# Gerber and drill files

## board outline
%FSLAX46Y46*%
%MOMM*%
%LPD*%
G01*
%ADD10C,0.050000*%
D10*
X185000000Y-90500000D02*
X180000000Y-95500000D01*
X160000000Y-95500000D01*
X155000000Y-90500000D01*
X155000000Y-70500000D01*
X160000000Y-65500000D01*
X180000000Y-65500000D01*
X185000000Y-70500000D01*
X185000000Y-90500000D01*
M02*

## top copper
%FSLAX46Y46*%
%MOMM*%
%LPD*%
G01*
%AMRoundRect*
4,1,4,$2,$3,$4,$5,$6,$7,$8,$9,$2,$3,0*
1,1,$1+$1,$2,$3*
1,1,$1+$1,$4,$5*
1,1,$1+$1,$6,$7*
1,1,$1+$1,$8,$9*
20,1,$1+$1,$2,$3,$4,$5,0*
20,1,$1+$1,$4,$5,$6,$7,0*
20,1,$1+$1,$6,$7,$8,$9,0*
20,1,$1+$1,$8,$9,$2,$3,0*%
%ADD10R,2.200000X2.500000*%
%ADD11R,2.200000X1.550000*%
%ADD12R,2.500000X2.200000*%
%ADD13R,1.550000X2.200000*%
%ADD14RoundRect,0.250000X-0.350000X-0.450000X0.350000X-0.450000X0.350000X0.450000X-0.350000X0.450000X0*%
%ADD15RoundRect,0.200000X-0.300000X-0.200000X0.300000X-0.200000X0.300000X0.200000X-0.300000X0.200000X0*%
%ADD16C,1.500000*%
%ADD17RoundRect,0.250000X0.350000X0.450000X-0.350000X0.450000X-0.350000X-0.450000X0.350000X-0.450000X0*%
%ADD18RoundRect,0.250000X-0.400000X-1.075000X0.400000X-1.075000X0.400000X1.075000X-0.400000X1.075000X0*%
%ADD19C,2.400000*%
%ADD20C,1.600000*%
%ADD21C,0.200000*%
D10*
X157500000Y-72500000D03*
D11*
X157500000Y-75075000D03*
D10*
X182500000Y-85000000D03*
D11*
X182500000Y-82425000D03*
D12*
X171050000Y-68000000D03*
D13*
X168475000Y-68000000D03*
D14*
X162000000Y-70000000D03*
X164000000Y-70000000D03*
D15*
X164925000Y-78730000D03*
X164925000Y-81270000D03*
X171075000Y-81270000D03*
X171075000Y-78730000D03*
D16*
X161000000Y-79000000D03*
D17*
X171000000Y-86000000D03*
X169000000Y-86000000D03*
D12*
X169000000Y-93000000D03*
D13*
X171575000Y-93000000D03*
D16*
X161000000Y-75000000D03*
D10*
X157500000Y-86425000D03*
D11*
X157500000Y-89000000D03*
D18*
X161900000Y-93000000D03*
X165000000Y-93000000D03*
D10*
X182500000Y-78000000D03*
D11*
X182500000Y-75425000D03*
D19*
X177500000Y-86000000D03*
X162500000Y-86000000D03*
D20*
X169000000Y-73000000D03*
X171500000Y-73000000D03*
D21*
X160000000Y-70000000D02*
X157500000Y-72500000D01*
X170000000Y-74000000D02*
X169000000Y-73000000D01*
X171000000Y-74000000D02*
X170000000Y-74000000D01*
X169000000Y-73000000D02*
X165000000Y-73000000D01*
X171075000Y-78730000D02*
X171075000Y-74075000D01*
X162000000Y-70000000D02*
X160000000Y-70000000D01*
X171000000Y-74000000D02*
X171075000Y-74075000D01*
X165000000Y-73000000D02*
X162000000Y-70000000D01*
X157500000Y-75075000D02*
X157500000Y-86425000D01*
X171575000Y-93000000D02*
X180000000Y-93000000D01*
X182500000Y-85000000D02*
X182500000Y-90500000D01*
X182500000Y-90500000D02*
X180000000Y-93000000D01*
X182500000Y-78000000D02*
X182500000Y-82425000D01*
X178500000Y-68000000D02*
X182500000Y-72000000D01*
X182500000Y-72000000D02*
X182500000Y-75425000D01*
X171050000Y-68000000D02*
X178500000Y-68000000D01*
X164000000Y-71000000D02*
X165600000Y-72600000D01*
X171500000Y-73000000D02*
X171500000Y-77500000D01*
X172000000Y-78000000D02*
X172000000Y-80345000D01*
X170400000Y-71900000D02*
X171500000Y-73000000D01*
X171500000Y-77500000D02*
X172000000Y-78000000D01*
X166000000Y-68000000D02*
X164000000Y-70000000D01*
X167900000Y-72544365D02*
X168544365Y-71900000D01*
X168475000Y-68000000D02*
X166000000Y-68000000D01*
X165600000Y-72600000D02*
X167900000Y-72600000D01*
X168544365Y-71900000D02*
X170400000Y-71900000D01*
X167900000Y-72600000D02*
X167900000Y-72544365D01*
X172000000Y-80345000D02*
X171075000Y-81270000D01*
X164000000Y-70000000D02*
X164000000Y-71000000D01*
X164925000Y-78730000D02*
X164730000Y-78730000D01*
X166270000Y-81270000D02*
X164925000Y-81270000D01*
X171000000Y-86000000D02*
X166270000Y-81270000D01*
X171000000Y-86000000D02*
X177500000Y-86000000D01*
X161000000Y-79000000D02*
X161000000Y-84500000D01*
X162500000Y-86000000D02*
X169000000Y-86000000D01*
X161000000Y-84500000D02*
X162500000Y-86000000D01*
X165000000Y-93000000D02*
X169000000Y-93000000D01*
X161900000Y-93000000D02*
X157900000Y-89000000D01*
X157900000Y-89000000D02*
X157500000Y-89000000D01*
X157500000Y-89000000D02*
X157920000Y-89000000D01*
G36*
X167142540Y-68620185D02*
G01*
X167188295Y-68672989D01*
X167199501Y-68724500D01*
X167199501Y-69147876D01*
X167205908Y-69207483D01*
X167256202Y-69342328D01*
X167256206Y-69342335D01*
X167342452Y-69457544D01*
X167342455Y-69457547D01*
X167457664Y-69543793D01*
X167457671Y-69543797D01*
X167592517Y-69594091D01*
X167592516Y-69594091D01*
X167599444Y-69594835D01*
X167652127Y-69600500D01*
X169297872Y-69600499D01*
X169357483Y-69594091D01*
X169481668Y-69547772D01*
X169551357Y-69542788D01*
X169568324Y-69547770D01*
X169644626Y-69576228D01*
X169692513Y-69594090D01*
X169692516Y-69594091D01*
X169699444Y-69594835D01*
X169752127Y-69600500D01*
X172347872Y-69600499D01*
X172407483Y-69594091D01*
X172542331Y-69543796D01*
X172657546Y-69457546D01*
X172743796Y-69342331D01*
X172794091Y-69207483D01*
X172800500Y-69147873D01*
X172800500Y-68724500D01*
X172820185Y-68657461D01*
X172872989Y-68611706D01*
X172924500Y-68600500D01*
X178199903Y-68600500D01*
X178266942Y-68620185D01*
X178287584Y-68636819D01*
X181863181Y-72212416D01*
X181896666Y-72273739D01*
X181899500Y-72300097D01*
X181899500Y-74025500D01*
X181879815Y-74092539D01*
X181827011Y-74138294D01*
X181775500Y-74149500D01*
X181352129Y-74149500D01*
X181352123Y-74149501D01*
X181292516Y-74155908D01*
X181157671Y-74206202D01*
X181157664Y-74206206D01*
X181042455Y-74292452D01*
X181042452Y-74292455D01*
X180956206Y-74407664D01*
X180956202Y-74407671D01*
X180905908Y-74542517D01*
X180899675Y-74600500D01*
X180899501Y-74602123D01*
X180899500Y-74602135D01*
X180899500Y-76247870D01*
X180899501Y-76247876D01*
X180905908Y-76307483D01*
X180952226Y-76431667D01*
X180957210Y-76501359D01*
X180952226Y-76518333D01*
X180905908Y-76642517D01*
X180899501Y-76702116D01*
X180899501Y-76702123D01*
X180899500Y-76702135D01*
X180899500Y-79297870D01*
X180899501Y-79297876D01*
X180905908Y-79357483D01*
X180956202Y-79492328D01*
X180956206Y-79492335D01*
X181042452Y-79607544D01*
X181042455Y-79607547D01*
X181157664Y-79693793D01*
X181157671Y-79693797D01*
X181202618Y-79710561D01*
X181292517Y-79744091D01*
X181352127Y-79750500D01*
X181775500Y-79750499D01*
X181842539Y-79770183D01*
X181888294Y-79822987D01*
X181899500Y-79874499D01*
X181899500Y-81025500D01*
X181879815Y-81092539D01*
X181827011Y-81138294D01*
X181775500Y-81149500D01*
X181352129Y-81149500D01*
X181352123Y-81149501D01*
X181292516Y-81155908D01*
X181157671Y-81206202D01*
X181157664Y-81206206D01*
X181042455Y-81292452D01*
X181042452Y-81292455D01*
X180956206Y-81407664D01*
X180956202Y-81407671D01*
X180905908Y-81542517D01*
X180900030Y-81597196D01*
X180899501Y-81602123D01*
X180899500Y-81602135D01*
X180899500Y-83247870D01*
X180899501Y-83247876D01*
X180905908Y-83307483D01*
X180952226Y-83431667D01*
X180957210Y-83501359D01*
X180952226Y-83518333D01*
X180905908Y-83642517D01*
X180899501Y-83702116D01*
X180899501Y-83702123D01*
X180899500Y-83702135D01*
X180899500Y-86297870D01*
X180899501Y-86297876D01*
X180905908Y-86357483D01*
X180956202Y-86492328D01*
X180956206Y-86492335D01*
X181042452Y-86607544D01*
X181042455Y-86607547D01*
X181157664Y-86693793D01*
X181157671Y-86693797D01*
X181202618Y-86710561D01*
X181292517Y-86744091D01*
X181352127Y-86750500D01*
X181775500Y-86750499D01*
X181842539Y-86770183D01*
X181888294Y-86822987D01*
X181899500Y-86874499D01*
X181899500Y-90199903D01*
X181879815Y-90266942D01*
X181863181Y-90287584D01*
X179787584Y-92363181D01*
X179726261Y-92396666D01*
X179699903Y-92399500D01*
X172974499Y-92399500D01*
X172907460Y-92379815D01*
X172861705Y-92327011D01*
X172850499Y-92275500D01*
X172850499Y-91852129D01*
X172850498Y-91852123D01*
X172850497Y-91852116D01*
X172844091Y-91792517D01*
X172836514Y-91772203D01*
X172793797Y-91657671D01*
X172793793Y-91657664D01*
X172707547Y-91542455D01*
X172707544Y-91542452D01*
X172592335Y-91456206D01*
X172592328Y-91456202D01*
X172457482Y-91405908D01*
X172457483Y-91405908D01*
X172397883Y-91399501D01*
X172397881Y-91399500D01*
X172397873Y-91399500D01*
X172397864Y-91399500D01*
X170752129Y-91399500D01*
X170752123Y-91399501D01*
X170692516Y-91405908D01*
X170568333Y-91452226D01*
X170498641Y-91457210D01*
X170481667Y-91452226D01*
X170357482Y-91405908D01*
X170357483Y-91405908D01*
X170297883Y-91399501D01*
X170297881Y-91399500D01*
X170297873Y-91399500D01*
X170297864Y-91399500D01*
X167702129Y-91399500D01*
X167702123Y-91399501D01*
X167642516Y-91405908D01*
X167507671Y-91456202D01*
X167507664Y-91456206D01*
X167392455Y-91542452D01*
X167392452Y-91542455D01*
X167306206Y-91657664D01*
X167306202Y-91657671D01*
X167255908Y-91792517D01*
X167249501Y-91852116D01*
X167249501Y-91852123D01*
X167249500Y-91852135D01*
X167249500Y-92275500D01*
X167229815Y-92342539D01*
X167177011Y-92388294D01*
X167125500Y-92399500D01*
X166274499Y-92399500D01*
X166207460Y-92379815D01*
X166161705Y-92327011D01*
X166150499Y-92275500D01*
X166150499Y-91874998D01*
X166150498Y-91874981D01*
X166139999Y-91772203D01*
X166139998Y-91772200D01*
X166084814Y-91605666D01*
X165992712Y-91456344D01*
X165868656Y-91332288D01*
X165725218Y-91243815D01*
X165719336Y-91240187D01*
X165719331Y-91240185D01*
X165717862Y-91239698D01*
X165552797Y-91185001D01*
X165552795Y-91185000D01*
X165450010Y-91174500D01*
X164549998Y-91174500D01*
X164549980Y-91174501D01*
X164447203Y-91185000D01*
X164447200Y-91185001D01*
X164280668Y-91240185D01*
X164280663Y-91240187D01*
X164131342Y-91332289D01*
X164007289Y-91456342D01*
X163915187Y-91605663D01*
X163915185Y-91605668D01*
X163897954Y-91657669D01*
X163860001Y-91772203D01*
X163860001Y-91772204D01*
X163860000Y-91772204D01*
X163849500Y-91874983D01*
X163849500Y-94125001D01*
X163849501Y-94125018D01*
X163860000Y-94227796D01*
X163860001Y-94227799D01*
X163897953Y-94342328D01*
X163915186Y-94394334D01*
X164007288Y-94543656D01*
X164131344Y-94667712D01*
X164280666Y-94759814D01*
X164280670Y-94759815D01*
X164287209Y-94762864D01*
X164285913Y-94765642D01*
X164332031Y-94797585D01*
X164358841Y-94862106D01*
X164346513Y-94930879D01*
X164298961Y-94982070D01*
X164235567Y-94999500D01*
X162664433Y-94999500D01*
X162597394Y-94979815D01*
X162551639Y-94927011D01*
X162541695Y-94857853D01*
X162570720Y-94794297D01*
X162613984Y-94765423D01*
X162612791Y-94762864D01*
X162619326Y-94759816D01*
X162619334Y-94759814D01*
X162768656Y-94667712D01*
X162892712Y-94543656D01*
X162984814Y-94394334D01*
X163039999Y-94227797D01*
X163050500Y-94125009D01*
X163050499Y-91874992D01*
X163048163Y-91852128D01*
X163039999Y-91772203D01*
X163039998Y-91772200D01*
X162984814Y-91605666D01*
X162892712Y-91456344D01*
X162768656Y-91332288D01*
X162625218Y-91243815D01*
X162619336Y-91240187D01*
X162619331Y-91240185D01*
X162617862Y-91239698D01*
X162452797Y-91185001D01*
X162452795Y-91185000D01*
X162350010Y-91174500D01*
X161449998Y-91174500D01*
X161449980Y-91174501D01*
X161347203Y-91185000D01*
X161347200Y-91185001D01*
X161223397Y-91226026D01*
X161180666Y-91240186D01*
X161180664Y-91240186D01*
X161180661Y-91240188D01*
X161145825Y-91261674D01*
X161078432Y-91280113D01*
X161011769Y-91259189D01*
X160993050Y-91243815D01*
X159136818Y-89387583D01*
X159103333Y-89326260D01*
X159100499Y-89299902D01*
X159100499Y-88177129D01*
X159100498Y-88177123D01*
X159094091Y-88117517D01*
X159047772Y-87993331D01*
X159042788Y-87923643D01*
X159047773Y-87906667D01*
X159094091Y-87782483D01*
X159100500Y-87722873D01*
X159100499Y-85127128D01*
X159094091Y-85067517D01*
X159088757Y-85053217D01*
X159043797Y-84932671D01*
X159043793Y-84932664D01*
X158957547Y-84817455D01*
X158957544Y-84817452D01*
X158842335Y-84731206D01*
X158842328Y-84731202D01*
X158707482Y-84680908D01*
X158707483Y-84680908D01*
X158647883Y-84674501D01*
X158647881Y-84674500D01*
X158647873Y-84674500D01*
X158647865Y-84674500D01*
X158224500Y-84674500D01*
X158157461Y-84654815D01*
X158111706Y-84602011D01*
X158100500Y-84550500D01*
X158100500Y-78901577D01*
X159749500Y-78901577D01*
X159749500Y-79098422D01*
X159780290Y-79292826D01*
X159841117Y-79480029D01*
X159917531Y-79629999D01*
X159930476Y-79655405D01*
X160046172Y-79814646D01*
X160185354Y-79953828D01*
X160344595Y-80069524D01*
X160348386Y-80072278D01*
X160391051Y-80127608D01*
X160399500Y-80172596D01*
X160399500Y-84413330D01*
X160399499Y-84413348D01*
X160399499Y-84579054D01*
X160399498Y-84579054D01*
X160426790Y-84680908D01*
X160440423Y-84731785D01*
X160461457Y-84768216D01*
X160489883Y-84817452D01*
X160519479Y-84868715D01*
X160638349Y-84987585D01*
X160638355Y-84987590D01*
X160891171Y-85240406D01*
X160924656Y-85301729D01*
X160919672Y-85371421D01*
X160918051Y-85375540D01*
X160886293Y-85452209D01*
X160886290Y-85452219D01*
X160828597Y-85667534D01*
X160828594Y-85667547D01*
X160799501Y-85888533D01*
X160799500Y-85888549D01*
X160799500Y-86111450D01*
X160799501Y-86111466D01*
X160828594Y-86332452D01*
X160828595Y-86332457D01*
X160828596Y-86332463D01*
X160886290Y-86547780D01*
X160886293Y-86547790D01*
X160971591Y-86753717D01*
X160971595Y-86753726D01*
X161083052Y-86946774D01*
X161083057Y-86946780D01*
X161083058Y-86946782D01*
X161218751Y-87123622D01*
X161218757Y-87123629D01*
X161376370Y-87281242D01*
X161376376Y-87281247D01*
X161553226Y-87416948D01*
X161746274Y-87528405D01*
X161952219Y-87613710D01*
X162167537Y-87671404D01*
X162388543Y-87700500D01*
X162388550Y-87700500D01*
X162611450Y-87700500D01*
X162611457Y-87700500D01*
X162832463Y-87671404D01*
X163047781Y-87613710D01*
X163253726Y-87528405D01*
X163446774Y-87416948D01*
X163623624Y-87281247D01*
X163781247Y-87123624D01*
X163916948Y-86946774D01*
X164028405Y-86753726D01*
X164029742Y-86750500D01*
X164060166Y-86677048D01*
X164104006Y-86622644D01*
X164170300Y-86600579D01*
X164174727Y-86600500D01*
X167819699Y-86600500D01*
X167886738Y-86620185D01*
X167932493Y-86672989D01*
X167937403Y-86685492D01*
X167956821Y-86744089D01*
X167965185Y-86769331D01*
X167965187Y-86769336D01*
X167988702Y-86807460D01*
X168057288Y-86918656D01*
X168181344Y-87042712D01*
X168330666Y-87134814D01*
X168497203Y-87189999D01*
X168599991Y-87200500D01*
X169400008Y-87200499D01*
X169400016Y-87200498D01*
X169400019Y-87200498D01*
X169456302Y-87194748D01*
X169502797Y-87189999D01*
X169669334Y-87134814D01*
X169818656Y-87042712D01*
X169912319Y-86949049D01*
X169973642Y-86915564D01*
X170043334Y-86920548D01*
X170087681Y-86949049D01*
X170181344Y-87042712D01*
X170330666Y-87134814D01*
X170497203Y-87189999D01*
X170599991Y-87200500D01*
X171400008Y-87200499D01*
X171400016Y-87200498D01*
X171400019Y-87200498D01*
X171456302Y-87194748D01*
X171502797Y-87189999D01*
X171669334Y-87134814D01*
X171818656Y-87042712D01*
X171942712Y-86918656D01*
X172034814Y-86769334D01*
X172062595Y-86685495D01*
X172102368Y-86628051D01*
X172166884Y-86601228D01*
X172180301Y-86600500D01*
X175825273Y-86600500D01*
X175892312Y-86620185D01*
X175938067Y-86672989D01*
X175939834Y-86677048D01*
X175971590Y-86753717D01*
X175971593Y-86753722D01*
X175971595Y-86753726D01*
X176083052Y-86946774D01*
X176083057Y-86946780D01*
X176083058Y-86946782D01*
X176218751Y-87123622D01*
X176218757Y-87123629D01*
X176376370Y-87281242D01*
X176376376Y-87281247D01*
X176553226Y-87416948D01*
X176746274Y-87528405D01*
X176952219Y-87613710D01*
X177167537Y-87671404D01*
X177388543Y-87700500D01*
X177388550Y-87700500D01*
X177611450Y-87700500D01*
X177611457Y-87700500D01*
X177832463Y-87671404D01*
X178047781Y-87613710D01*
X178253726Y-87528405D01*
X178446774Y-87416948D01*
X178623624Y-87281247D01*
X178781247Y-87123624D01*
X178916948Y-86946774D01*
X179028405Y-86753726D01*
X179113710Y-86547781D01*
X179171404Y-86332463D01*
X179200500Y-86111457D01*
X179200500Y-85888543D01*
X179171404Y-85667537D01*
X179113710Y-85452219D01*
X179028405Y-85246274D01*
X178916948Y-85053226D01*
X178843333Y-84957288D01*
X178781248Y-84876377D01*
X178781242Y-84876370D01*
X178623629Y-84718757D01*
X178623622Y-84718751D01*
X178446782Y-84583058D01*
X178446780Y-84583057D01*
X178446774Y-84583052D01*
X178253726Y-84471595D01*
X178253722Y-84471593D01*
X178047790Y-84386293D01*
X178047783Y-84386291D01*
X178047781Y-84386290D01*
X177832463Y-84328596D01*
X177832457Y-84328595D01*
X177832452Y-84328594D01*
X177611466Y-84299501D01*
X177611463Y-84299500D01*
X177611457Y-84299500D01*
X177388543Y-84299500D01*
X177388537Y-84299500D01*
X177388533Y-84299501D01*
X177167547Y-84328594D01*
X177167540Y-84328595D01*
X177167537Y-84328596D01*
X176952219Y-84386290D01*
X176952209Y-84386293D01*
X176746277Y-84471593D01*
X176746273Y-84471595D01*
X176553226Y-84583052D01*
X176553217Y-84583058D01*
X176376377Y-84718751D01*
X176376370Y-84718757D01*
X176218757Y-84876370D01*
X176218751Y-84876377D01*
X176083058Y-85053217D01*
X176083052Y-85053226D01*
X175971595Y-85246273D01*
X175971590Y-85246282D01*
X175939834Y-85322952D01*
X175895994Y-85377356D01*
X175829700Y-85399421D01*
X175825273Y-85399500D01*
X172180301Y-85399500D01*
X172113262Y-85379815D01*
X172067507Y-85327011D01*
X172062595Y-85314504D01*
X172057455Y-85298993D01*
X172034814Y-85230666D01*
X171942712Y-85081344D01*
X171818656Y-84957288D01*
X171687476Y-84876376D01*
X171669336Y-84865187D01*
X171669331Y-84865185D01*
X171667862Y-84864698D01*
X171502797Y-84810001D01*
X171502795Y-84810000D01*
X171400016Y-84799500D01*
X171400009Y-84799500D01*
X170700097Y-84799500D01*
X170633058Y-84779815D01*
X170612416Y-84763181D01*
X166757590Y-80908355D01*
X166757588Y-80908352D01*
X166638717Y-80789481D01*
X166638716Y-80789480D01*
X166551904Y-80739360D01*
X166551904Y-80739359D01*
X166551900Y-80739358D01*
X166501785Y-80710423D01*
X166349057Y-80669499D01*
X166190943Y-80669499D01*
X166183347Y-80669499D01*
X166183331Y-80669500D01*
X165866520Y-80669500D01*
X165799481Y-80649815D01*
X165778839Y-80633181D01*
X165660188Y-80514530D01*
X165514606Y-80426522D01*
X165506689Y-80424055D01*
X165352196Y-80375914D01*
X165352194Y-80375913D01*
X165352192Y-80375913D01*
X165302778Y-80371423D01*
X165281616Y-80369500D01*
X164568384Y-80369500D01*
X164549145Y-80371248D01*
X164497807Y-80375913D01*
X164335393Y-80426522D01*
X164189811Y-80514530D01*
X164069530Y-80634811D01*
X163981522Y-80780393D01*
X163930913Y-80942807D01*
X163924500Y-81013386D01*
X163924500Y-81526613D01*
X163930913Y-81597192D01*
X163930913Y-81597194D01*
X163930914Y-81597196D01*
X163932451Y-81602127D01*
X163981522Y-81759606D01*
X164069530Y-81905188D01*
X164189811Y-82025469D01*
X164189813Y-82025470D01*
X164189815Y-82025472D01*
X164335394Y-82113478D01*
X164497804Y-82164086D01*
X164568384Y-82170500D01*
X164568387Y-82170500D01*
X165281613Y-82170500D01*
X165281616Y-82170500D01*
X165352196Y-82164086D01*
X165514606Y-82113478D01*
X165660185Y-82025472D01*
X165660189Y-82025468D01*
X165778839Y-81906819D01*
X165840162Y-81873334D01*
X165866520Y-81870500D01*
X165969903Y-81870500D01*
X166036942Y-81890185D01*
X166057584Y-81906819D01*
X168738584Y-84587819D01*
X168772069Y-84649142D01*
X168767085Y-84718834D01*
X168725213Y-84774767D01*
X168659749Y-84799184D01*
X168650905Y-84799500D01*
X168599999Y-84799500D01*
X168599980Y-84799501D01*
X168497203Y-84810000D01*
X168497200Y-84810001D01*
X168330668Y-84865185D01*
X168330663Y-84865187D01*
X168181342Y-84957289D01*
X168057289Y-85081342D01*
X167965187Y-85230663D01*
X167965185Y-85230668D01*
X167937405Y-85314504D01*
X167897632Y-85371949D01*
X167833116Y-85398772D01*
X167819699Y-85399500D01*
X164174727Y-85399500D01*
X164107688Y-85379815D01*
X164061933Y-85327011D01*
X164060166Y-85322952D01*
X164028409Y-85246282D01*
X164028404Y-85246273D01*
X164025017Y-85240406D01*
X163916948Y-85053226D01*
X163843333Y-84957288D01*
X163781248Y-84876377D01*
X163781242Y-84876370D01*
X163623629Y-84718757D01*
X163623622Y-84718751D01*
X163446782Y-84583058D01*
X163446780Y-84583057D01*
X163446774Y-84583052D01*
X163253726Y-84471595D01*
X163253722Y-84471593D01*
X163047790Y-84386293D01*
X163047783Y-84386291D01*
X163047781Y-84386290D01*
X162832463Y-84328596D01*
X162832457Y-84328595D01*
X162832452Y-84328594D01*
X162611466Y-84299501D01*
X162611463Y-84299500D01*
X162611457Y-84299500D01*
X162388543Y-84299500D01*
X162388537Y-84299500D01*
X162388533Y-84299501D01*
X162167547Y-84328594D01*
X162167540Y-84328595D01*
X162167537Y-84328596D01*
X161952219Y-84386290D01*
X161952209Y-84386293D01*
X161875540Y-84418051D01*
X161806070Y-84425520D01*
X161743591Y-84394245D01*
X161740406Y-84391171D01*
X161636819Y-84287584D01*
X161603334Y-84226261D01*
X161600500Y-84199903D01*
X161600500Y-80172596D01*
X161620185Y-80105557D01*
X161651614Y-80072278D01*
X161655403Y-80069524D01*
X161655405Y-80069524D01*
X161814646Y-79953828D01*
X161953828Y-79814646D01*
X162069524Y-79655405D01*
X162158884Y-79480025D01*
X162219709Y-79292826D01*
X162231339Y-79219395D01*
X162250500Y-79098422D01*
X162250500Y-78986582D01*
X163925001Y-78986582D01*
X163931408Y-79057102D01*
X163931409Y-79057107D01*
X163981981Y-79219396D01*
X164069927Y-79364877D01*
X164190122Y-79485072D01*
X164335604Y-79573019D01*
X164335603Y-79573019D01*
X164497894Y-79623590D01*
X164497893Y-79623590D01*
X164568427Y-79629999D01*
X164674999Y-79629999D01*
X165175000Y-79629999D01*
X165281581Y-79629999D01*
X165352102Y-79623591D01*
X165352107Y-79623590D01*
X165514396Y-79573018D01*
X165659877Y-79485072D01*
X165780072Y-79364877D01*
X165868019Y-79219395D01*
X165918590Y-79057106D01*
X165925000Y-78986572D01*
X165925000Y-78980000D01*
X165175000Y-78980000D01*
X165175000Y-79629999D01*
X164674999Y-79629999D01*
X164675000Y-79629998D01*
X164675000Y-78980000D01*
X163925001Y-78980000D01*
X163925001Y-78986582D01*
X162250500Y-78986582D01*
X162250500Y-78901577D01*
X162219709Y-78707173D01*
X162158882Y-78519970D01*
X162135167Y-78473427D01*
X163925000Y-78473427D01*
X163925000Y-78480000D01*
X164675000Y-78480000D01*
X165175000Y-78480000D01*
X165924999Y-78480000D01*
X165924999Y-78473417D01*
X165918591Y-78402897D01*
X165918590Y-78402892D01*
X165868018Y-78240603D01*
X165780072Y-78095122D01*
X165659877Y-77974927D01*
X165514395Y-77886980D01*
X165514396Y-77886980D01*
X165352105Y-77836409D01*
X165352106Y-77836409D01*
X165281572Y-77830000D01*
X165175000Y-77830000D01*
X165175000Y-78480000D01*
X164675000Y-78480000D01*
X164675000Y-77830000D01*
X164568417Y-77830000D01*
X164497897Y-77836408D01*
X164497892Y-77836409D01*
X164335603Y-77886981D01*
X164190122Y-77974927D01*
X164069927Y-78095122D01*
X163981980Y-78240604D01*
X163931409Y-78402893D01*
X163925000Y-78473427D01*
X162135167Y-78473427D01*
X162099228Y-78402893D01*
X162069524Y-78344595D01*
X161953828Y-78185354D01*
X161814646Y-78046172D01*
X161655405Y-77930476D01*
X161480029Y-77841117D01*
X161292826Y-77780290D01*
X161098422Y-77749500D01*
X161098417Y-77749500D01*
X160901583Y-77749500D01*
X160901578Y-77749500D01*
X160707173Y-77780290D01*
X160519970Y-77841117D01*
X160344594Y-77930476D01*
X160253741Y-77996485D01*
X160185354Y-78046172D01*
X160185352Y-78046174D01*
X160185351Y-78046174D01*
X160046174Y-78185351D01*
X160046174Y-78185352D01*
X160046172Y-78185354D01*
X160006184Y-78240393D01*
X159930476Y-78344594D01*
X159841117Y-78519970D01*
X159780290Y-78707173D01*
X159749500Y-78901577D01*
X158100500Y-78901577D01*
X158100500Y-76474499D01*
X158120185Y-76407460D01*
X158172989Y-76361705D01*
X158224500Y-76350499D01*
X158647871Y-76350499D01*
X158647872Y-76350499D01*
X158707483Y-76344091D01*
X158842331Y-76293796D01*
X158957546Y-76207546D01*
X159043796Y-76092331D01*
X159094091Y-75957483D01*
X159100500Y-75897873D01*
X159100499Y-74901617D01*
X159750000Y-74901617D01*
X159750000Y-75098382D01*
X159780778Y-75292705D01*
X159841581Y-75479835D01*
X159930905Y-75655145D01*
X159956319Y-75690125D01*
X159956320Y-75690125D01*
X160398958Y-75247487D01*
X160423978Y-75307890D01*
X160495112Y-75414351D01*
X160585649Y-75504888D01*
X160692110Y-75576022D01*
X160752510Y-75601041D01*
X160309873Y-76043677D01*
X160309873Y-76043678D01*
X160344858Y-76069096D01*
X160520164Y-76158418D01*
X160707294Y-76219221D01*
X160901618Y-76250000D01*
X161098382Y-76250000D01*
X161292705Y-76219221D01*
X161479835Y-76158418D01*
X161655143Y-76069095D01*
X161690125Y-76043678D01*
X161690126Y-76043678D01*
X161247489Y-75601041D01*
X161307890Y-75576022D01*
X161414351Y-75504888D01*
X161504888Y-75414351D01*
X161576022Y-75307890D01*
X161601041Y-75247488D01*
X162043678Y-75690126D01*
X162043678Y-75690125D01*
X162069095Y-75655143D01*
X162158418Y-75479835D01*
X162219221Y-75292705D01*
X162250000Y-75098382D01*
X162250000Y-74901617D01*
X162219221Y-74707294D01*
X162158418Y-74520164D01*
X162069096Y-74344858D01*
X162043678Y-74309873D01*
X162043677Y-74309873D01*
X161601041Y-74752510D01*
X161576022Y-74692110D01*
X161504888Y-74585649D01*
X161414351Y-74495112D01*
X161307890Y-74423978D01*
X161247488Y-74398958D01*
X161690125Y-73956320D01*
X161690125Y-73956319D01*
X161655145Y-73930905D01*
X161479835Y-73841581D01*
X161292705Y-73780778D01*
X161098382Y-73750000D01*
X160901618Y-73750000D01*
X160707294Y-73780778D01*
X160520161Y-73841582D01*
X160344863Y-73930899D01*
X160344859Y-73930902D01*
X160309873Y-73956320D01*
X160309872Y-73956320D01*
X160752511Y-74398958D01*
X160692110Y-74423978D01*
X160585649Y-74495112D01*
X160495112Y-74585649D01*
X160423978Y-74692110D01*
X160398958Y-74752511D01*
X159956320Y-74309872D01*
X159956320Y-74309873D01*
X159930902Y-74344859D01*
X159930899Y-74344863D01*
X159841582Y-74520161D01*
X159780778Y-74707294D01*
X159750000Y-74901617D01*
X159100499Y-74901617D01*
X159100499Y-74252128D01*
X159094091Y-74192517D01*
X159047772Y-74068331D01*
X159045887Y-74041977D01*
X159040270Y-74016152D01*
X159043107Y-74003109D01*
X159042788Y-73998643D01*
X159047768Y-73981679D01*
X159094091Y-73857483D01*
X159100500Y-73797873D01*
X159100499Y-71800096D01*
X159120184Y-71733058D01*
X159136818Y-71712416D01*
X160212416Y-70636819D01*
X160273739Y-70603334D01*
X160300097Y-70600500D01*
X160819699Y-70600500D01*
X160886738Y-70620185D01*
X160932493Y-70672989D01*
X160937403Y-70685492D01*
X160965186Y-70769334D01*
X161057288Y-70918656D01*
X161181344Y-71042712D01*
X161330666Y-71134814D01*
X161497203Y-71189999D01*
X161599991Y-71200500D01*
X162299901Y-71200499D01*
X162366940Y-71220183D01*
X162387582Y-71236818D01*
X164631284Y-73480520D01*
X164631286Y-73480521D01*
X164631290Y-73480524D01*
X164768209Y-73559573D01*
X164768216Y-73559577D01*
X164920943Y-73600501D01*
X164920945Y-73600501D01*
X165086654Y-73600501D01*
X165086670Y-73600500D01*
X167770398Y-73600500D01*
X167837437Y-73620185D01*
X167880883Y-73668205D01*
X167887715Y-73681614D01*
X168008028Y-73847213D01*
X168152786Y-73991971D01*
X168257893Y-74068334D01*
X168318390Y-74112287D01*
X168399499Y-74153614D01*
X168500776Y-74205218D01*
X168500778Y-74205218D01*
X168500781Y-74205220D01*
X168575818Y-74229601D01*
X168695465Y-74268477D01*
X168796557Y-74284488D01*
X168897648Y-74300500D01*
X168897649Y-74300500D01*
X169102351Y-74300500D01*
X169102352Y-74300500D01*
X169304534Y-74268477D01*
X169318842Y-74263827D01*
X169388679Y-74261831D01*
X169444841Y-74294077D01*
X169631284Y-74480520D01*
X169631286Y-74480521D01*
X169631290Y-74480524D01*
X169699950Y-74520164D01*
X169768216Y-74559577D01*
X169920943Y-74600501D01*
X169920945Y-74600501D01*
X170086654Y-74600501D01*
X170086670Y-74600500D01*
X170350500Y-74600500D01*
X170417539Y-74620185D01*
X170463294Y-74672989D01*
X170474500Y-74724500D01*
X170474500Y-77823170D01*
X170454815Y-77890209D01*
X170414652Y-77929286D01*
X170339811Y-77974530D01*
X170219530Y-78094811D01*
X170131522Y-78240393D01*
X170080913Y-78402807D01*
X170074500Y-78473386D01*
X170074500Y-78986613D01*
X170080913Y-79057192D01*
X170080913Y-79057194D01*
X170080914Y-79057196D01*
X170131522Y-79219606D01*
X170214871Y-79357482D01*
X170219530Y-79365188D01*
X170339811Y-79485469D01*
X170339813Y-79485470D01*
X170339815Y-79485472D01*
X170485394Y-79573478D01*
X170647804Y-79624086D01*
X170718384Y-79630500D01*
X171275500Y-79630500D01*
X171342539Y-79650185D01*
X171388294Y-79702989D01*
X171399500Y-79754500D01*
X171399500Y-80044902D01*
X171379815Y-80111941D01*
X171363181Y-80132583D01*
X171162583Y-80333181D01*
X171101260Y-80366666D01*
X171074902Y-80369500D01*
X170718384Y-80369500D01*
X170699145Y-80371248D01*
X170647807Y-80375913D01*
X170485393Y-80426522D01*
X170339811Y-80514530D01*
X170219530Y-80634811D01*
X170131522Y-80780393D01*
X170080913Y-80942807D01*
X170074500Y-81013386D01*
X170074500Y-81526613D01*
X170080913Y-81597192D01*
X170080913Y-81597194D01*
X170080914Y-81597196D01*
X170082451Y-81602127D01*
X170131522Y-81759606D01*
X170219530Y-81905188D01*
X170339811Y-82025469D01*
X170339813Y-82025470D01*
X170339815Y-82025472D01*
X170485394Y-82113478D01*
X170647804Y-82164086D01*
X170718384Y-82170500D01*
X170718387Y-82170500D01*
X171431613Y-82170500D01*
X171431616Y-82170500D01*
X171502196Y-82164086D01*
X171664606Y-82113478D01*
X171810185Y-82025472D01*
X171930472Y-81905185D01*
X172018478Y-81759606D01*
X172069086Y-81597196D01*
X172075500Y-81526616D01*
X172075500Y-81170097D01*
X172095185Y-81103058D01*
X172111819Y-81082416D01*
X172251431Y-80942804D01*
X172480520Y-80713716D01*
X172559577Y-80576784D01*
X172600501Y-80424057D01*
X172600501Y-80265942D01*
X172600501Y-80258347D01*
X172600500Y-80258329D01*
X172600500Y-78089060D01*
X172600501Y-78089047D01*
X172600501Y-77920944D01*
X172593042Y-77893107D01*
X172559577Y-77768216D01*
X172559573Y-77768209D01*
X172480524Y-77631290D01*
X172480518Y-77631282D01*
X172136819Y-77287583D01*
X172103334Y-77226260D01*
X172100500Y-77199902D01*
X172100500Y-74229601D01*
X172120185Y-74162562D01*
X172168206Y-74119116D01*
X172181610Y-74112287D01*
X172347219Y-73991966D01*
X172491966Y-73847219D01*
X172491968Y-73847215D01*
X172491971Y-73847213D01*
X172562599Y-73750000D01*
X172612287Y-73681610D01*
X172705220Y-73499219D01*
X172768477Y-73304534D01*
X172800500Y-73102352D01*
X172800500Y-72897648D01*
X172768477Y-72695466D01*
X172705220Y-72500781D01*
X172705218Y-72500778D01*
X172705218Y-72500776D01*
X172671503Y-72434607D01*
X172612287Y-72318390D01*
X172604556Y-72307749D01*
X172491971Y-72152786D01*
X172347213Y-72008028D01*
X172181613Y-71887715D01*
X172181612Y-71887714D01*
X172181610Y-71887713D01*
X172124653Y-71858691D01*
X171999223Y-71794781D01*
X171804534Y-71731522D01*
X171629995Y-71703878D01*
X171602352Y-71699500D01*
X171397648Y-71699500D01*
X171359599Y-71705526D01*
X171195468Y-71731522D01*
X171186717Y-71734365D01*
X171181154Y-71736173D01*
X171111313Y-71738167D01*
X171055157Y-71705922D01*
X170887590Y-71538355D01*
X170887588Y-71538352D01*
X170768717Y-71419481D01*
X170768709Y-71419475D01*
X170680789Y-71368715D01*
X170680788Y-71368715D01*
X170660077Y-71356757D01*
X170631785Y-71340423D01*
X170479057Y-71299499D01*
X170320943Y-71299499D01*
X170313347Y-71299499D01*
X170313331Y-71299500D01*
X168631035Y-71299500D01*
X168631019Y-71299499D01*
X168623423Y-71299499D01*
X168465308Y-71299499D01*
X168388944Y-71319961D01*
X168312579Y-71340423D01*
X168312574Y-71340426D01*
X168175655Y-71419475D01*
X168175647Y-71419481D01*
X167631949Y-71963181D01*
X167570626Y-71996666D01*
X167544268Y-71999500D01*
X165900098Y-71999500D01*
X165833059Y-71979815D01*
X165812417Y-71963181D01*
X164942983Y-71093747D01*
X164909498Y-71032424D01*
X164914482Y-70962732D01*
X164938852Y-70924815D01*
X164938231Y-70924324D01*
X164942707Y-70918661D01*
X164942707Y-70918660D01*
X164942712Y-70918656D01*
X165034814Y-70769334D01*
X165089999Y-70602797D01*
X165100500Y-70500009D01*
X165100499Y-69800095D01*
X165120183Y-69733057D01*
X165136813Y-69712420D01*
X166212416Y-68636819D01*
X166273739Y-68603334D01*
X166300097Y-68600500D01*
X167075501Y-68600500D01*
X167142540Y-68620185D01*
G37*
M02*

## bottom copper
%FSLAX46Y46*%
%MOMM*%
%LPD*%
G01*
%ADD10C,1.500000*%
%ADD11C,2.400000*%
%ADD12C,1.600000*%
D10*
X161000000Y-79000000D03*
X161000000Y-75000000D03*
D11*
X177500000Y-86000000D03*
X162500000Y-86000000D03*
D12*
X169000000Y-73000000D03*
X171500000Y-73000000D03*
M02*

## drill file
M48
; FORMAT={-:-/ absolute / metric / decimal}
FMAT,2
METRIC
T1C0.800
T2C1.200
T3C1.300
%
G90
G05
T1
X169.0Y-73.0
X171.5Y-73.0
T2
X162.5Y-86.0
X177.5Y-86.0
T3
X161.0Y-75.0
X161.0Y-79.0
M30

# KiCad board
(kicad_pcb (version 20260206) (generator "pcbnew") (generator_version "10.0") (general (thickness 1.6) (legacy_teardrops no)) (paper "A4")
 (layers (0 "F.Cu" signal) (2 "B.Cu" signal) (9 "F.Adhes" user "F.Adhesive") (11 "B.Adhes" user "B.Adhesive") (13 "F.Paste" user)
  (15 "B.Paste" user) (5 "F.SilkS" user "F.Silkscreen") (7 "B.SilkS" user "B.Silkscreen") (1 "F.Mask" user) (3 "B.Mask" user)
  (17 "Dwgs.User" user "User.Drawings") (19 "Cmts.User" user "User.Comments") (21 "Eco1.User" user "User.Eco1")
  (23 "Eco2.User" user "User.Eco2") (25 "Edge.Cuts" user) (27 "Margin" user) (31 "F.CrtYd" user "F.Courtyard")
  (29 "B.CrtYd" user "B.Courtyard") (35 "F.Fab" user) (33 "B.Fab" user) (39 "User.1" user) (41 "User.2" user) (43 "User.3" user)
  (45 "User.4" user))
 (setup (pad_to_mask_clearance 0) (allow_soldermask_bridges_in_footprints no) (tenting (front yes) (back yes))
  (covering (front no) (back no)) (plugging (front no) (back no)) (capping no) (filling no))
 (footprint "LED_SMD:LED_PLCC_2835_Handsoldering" (layer "F.Cu") (at 157.5 73.55 -90)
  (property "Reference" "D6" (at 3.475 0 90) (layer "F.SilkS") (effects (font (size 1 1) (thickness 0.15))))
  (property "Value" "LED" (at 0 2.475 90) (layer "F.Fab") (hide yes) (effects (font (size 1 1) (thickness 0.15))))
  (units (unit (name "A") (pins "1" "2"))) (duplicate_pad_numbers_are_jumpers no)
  (pad "1" smd rect (at -1.05 0 270) (size 2.5 2.2) (layers "F.Cu" "F.Mask" "F.Paste") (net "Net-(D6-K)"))
  (pad "2" smd rect (at 1.525 0 270) (size 1.55 2.2) (layers "F.Cu" "F.Mask" "F.Paste") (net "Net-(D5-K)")))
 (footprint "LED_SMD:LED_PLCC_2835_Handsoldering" (layer "F.Cu") (at 182.5 83.95 90)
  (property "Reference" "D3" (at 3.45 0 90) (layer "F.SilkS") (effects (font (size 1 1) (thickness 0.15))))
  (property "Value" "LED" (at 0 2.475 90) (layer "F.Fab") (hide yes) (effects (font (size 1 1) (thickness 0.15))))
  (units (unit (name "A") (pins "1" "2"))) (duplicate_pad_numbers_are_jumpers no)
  (pad "1" smd rect (at -1.05 0 90) (size 2.5 2.2) (layers "F.Cu" "F.Mask" "F.Paste") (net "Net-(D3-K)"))
  (pad "2" smd rect (at 1.525 0 90) (size 1.55 2.2) (layers "F.Cu" "F.Mask" "F.Paste") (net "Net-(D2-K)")))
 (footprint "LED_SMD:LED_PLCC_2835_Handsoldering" (layer "F.Cu") (at 170 68 180)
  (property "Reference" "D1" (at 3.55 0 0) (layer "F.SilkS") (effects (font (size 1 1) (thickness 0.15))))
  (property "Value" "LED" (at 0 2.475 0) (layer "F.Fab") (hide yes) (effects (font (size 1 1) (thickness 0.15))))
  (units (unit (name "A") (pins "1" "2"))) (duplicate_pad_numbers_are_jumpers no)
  (pad "1" smd rect (at -1.05 0 180) (size 2.5 2.2) (layers "F.Cu" "F.Mask" "F.Paste") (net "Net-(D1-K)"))
  (pad "2" smd rect (at 1.525 0 180) (size 1.55 2.2) (layers "F.Cu" "F.Mask" "F.Paste") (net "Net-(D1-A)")))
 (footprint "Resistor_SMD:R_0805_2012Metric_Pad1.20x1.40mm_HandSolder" (layer "F.Cu") (at 163 70)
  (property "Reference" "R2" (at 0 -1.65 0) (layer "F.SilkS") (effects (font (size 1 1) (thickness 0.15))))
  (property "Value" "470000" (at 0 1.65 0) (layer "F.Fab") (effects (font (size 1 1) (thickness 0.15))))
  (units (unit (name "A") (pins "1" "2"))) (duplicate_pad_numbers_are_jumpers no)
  (pad "1" smd roundrect (at -1 0) (size 1.2 1.4) (layers "F.Cu" "F.Mask" "F.Paste") (roundrect_rratio 0.208333) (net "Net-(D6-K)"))
  (pad "2" smd roundrect (at 1 0) (size 1.2 1.4) (layers "F.Cu" "F.Mask" "F.Paste") (roundrect_rratio 0.208333) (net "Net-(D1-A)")))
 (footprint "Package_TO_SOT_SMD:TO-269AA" (layer "F.Cu") (at 168 80)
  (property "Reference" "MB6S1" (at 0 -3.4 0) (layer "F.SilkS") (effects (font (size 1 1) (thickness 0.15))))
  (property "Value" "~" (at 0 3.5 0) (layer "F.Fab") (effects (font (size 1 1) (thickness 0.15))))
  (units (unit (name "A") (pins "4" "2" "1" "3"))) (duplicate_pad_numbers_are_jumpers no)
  (pad "1" smd roundrect (at -3.075 -1.27) (size 1 0.8) (layers "F.Cu" "F.Mask" "F.Paste") (roundrect_rratio 0.25) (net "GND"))
  (pad "2" smd roundrect (at -3.075 1.27) (size 1 0.8) (layers "F.Cu" "F.Mask" "F.Paste") (roundrect_rratio 0.25) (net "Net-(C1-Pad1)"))
  (pad "3" smd roundrect (at 3.075 1.27) (size 1 0.8) (layers "F.Cu" "F.Mask" "F.Paste") (roundrect_rratio 0.25) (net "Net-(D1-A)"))
  (pad "4" smd roundrect (at 3.075 -1.27) (size 1 0.8) (layers "F.Cu" "F.Mask" "F.Paste") (roundrect_rratio 0.25) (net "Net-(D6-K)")))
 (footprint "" (layer "F.Cu") (at 161 79)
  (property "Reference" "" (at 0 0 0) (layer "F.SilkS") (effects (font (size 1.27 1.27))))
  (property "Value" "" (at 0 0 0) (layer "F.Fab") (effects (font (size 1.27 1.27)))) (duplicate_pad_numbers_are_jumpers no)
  (pad "power" thru_hole circle (at 0 0) (size 1.5 1.5) (drill 1.3) (layers "*.Cu" "*.Mask") (remove_unused_layers no) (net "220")))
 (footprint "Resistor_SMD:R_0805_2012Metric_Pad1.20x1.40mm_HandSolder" (layer "F.Cu") (at 170 86 180)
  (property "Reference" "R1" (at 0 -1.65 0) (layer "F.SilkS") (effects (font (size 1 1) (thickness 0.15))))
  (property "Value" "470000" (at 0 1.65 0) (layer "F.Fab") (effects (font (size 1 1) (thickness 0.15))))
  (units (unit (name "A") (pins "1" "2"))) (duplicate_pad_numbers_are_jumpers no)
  (pad "1" smd roundrect (at -1 0 180) (size 1.2 1.4) (layers "F.Cu" "F.Mask" "F.Paste") (roundrect_rratio 0.208333) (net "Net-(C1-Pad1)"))
  (pad "2" smd roundrect (at 1 0 180) (size 1.2 1.4) (layers "F.Cu" "F.Mask" "F.Paste") (roundrect_rratio 0.208333) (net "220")))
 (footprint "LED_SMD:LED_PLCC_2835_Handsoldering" (layer "F.Cu") (at 170.05 93)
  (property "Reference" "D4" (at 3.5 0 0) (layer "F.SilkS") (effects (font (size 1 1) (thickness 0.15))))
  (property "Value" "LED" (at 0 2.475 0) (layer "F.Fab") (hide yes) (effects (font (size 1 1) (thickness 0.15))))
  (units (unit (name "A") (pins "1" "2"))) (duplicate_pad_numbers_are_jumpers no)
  (pad "1" smd rect (at -1.05 0) (size 2.5 2.2) (layers "F.Cu" "F.Mask" "F.Paste") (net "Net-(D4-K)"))
  (pad "2" smd rect (at 1.525 0) (size 1.55 2.2) (layers "F.Cu" "F.Mask" "F.Paste") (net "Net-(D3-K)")))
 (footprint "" (layer "F.Cu") (at 161 75)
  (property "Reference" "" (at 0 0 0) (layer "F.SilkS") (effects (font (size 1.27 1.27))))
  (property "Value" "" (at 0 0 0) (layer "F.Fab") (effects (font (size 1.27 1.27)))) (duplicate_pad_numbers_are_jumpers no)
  (pad "1" thru_hole circle (at 0 0) (size 1.5 1.5) (drill 1.3) (layers "*.Cu" "*.Mask") (remove_unused_layers no) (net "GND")))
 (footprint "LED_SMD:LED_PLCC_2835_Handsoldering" (layer "F.Cu") (at 157.5 87.475 -90)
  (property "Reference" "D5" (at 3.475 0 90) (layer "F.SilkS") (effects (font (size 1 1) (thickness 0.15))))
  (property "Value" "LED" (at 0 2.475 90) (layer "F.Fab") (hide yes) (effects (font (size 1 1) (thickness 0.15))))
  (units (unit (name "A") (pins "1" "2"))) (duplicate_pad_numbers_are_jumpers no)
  (pad "1" smd rect (at -1.05 0 270) (size 2.5 2.2) (layers "F.Cu" "F.Mask" "F.Paste") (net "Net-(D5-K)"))
  (pad "2" smd rect (at 1.525 0 270) (size 1.55 2.2) (layers "F.Cu" "F.Mask" "F.Paste") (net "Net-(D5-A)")))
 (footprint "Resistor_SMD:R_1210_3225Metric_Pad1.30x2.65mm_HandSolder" (layer "F.Cu") (at 163.45 93)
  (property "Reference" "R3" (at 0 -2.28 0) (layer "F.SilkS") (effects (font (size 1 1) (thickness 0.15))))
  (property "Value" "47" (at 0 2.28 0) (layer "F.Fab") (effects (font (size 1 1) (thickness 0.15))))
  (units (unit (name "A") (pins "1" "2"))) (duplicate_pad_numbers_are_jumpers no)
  (pad "1" smd roundrect (at -1.55 0) (size 1.3 2.65) (layers "F.Cu" "F.Mask" "F.Paste") (roundrect_rratio 0.192308) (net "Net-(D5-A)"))
  (pad "2" smd roundrect (at 1.55 0) (size 1.3 2.65) (layers "F.Cu" "F.Mask" "F.Paste") (roundrect_rratio 0.192308) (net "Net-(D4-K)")))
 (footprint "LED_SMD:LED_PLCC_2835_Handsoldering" (layer "F.Cu") (at 182.5 76.95 90)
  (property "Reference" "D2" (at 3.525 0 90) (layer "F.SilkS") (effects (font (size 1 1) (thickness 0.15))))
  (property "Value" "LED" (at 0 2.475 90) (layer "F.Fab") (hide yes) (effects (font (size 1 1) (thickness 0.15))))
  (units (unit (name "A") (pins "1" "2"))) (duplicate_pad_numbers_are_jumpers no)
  (pad "1" smd rect (at -1.05 0 90) (size 2.5 2.2) (layers "F.Cu" "F.Mask" "F.Paste") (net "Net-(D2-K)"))
  (pad "2" smd rect (at 1.525 0 90) (size 1.55 2.2) (layers "F.Cu" "F.Mask" "F.Paste") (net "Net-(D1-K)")))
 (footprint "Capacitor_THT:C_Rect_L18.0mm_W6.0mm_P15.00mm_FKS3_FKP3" (layer "B.Cu") (at 177.5 86 180)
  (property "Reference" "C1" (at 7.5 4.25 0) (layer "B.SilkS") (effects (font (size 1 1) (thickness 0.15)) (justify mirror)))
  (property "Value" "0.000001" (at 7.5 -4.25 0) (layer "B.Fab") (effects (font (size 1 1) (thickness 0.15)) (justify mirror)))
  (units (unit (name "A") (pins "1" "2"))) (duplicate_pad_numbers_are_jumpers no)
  (pad "1" thru_hole circle (at 0 0 180) (size 2.4 2.4) (drill 1.2) (layers "*.Cu" "*.Mask") (remove_unused_layers no) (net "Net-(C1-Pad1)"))
  (pad "2" thru_hole circle (at 15 0 180) (size 2.4 2.4) (drill 1.2) (layers "*.Cu" "*.Mask") (remove_unused_layers no) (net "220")))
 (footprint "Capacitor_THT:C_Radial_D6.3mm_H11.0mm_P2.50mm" (layer "B.Cu") (at 169 73)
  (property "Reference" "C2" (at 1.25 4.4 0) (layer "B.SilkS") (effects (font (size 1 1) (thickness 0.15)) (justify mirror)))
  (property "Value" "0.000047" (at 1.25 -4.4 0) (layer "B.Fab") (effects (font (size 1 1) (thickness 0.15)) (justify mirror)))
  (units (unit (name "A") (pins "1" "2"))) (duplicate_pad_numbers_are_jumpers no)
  (pad "1" thru_hole circle (at 0 0) (size 1.6 1.6) (drill 0.8) (layers "*.Cu" "*.Mask") (remove_unused_layers no) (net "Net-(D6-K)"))
  (pad "2" thru_hole circle (at 2.5 0) (size 1.6 1.6) (drill 0.8) (layers "*.Cu" "*.Mask") (remove_unused_layers no) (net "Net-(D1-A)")))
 (gr_poly
  (pts (xy 185 90.5) (xy 180 95.5) (xy 160 95.5) (xy 155 90.5) (xy 155 70.5) (xy 160 65.5) (xy 180 65.5) (xy 185 70.5))
  (stroke (width 0.05) (type solid)) (fill no) (layer "Edge.Cuts"))
 (segment (start 160 70) (end 157.5 72.5) (width 0.2) (layer "F.Cu") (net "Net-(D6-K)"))
 (segment (start 170 74) (end 169 73) (width 0.2) (layer "F.Cu") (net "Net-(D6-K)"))
 (segment (start 171 74) (end 170 74) (width 0.2) (layer "F.Cu") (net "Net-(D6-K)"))
 (segment (start 169 73) (end 165 73) (width 0.2) (layer "F.Cu") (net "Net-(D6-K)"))
 (segment (start 171.075 78.73) (end 171.075 74.075) (width 0.2) (layer "F.Cu") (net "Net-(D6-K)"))
 (segment (start 162 70) (end 160 70) (width 0.2) (layer "F.Cu") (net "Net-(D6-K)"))
 (segment (start 171 74) (end 171.075 74.075) (width 0.2) (layer "F.Cu") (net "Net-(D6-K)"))
 (segment (start 165 73) (end 162 70) (width 0.2) (layer "F.Cu") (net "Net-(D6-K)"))
 (segment (start 157.5 75.075) (end 157.5 86.425) (width 0.2) (layer "F.Cu") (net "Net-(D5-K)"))
 (segment (start 171.575 93) (end 180 93) (width 0.2) (layer "F.Cu") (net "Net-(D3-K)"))
 (segment (start 182.5 85) (end 182.5 90.5) (width 0.2) (layer "F.Cu") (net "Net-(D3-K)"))
 (segment (start 182.5 90.5) (end 180 93) (width 0.2) (layer "F.Cu") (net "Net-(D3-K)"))
 (segment (start 182.5 78) (end 182.5 82.425) (width 0.2) (layer "F.Cu") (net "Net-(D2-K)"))
 (segment (start 178.5 68) (end 182.5 72) (width 0.2) (layer "F.Cu") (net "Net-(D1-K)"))
 (segment (start 182.5 72) (end 182.5 75.425) (width 0.2) (layer "F.Cu") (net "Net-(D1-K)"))
 (segment (start 171.05 68) (end 178.5 68) (width 0.2) (layer "F.Cu") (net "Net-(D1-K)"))
 (segment (start 164 71) (end 165.6 72.6) (width 0.2) (layer "F.Cu") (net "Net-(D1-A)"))
 (segment (start 171.5 73) (end 171.5 77.5) (width 0.2) (layer "F.Cu") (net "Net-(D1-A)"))
 (segment (start 172 78) (end 172 80.345) (width 0.2) (layer "F.Cu") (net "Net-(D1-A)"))
 (segment (start 170.4 71.9) (end 171.5 73) (width 0.2) (layer "F.Cu") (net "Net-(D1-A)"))
 (segment (start 171.5 77.5) (end 172 78) (width 0.2) (layer "F.Cu") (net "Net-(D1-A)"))
 (segment (start 166 68) (end 164 70) (width 0.2) (layer "F.Cu") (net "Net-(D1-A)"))
 (segment (start 167.9 72.544365) (end 168.544365 71.9) (width 0.2) (layer "F.Cu") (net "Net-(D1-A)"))
 (segment (start 168.475 68) (end 166 68) (width 0.2) (layer "F.Cu") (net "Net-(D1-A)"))
 (segment (start 165.6 72.6) (end 167.9 72.6) (width 0.2) (layer "F.Cu") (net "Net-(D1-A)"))
 (segment (start 168.544365 71.9) (end 170.4 71.9) (width 0.2) (layer "F.Cu") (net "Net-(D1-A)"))
 (segment (start 167.9 72.6) (end 167.9 72.544365) (width 0.2) (layer "F.Cu") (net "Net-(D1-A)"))
 (segment (start 172 80.345) (end 171.075 81.27) (width 0.2) (layer "F.Cu") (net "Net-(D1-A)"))
 (segment (start 164 70) (end 164 71) (width 0.2) (layer "F.Cu") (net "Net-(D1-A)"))
 (segment (start 164.925 78.73) (end 164.73 78.73) (width 0.2) (layer "F.Cu") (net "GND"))
 (segment (start 166.27 81.27) (end 164.925 81.27) (width 0.2) (layer "F.Cu") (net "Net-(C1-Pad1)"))
 (segment (start 171 86) (end 166.27 81.27) (width 0.2) (layer "F.Cu") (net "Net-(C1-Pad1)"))
 (segment (start 171 86) (end 177.5 86) (width 0.2) (layer "F.Cu") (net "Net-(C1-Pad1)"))
 (segment (start 161 79) (end 161 84.5) (width 0.2) (layer "F.Cu") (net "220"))
 (segment (start 162.5 86) (end 169 86) (width 0.2) (layer "F.Cu") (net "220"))
 (segment (start 161 84.5) (end 162.5 86) (width 0.2) (layer "F.Cu") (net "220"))
 (segment (start 165 93) (end 169 93) (width 0.2) (layer "F.Cu") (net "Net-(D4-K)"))
 (segment (start 161.9 93) (end 157.9 89) (width 0.2) (layer "F.Cu") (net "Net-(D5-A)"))
 (segment (start 157.9 89) (end 157.5 89) (width 0.2) (layer "F.Cu") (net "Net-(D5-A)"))
 (segment (start 157.5 89) (end 157.92 89) (width 0.2) (layer "F.Cu") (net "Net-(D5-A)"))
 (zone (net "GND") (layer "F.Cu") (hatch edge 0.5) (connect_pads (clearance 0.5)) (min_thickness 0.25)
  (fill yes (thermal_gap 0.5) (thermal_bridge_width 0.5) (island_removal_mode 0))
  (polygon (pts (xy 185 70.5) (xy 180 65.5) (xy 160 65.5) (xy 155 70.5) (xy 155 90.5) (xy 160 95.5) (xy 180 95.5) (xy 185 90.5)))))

